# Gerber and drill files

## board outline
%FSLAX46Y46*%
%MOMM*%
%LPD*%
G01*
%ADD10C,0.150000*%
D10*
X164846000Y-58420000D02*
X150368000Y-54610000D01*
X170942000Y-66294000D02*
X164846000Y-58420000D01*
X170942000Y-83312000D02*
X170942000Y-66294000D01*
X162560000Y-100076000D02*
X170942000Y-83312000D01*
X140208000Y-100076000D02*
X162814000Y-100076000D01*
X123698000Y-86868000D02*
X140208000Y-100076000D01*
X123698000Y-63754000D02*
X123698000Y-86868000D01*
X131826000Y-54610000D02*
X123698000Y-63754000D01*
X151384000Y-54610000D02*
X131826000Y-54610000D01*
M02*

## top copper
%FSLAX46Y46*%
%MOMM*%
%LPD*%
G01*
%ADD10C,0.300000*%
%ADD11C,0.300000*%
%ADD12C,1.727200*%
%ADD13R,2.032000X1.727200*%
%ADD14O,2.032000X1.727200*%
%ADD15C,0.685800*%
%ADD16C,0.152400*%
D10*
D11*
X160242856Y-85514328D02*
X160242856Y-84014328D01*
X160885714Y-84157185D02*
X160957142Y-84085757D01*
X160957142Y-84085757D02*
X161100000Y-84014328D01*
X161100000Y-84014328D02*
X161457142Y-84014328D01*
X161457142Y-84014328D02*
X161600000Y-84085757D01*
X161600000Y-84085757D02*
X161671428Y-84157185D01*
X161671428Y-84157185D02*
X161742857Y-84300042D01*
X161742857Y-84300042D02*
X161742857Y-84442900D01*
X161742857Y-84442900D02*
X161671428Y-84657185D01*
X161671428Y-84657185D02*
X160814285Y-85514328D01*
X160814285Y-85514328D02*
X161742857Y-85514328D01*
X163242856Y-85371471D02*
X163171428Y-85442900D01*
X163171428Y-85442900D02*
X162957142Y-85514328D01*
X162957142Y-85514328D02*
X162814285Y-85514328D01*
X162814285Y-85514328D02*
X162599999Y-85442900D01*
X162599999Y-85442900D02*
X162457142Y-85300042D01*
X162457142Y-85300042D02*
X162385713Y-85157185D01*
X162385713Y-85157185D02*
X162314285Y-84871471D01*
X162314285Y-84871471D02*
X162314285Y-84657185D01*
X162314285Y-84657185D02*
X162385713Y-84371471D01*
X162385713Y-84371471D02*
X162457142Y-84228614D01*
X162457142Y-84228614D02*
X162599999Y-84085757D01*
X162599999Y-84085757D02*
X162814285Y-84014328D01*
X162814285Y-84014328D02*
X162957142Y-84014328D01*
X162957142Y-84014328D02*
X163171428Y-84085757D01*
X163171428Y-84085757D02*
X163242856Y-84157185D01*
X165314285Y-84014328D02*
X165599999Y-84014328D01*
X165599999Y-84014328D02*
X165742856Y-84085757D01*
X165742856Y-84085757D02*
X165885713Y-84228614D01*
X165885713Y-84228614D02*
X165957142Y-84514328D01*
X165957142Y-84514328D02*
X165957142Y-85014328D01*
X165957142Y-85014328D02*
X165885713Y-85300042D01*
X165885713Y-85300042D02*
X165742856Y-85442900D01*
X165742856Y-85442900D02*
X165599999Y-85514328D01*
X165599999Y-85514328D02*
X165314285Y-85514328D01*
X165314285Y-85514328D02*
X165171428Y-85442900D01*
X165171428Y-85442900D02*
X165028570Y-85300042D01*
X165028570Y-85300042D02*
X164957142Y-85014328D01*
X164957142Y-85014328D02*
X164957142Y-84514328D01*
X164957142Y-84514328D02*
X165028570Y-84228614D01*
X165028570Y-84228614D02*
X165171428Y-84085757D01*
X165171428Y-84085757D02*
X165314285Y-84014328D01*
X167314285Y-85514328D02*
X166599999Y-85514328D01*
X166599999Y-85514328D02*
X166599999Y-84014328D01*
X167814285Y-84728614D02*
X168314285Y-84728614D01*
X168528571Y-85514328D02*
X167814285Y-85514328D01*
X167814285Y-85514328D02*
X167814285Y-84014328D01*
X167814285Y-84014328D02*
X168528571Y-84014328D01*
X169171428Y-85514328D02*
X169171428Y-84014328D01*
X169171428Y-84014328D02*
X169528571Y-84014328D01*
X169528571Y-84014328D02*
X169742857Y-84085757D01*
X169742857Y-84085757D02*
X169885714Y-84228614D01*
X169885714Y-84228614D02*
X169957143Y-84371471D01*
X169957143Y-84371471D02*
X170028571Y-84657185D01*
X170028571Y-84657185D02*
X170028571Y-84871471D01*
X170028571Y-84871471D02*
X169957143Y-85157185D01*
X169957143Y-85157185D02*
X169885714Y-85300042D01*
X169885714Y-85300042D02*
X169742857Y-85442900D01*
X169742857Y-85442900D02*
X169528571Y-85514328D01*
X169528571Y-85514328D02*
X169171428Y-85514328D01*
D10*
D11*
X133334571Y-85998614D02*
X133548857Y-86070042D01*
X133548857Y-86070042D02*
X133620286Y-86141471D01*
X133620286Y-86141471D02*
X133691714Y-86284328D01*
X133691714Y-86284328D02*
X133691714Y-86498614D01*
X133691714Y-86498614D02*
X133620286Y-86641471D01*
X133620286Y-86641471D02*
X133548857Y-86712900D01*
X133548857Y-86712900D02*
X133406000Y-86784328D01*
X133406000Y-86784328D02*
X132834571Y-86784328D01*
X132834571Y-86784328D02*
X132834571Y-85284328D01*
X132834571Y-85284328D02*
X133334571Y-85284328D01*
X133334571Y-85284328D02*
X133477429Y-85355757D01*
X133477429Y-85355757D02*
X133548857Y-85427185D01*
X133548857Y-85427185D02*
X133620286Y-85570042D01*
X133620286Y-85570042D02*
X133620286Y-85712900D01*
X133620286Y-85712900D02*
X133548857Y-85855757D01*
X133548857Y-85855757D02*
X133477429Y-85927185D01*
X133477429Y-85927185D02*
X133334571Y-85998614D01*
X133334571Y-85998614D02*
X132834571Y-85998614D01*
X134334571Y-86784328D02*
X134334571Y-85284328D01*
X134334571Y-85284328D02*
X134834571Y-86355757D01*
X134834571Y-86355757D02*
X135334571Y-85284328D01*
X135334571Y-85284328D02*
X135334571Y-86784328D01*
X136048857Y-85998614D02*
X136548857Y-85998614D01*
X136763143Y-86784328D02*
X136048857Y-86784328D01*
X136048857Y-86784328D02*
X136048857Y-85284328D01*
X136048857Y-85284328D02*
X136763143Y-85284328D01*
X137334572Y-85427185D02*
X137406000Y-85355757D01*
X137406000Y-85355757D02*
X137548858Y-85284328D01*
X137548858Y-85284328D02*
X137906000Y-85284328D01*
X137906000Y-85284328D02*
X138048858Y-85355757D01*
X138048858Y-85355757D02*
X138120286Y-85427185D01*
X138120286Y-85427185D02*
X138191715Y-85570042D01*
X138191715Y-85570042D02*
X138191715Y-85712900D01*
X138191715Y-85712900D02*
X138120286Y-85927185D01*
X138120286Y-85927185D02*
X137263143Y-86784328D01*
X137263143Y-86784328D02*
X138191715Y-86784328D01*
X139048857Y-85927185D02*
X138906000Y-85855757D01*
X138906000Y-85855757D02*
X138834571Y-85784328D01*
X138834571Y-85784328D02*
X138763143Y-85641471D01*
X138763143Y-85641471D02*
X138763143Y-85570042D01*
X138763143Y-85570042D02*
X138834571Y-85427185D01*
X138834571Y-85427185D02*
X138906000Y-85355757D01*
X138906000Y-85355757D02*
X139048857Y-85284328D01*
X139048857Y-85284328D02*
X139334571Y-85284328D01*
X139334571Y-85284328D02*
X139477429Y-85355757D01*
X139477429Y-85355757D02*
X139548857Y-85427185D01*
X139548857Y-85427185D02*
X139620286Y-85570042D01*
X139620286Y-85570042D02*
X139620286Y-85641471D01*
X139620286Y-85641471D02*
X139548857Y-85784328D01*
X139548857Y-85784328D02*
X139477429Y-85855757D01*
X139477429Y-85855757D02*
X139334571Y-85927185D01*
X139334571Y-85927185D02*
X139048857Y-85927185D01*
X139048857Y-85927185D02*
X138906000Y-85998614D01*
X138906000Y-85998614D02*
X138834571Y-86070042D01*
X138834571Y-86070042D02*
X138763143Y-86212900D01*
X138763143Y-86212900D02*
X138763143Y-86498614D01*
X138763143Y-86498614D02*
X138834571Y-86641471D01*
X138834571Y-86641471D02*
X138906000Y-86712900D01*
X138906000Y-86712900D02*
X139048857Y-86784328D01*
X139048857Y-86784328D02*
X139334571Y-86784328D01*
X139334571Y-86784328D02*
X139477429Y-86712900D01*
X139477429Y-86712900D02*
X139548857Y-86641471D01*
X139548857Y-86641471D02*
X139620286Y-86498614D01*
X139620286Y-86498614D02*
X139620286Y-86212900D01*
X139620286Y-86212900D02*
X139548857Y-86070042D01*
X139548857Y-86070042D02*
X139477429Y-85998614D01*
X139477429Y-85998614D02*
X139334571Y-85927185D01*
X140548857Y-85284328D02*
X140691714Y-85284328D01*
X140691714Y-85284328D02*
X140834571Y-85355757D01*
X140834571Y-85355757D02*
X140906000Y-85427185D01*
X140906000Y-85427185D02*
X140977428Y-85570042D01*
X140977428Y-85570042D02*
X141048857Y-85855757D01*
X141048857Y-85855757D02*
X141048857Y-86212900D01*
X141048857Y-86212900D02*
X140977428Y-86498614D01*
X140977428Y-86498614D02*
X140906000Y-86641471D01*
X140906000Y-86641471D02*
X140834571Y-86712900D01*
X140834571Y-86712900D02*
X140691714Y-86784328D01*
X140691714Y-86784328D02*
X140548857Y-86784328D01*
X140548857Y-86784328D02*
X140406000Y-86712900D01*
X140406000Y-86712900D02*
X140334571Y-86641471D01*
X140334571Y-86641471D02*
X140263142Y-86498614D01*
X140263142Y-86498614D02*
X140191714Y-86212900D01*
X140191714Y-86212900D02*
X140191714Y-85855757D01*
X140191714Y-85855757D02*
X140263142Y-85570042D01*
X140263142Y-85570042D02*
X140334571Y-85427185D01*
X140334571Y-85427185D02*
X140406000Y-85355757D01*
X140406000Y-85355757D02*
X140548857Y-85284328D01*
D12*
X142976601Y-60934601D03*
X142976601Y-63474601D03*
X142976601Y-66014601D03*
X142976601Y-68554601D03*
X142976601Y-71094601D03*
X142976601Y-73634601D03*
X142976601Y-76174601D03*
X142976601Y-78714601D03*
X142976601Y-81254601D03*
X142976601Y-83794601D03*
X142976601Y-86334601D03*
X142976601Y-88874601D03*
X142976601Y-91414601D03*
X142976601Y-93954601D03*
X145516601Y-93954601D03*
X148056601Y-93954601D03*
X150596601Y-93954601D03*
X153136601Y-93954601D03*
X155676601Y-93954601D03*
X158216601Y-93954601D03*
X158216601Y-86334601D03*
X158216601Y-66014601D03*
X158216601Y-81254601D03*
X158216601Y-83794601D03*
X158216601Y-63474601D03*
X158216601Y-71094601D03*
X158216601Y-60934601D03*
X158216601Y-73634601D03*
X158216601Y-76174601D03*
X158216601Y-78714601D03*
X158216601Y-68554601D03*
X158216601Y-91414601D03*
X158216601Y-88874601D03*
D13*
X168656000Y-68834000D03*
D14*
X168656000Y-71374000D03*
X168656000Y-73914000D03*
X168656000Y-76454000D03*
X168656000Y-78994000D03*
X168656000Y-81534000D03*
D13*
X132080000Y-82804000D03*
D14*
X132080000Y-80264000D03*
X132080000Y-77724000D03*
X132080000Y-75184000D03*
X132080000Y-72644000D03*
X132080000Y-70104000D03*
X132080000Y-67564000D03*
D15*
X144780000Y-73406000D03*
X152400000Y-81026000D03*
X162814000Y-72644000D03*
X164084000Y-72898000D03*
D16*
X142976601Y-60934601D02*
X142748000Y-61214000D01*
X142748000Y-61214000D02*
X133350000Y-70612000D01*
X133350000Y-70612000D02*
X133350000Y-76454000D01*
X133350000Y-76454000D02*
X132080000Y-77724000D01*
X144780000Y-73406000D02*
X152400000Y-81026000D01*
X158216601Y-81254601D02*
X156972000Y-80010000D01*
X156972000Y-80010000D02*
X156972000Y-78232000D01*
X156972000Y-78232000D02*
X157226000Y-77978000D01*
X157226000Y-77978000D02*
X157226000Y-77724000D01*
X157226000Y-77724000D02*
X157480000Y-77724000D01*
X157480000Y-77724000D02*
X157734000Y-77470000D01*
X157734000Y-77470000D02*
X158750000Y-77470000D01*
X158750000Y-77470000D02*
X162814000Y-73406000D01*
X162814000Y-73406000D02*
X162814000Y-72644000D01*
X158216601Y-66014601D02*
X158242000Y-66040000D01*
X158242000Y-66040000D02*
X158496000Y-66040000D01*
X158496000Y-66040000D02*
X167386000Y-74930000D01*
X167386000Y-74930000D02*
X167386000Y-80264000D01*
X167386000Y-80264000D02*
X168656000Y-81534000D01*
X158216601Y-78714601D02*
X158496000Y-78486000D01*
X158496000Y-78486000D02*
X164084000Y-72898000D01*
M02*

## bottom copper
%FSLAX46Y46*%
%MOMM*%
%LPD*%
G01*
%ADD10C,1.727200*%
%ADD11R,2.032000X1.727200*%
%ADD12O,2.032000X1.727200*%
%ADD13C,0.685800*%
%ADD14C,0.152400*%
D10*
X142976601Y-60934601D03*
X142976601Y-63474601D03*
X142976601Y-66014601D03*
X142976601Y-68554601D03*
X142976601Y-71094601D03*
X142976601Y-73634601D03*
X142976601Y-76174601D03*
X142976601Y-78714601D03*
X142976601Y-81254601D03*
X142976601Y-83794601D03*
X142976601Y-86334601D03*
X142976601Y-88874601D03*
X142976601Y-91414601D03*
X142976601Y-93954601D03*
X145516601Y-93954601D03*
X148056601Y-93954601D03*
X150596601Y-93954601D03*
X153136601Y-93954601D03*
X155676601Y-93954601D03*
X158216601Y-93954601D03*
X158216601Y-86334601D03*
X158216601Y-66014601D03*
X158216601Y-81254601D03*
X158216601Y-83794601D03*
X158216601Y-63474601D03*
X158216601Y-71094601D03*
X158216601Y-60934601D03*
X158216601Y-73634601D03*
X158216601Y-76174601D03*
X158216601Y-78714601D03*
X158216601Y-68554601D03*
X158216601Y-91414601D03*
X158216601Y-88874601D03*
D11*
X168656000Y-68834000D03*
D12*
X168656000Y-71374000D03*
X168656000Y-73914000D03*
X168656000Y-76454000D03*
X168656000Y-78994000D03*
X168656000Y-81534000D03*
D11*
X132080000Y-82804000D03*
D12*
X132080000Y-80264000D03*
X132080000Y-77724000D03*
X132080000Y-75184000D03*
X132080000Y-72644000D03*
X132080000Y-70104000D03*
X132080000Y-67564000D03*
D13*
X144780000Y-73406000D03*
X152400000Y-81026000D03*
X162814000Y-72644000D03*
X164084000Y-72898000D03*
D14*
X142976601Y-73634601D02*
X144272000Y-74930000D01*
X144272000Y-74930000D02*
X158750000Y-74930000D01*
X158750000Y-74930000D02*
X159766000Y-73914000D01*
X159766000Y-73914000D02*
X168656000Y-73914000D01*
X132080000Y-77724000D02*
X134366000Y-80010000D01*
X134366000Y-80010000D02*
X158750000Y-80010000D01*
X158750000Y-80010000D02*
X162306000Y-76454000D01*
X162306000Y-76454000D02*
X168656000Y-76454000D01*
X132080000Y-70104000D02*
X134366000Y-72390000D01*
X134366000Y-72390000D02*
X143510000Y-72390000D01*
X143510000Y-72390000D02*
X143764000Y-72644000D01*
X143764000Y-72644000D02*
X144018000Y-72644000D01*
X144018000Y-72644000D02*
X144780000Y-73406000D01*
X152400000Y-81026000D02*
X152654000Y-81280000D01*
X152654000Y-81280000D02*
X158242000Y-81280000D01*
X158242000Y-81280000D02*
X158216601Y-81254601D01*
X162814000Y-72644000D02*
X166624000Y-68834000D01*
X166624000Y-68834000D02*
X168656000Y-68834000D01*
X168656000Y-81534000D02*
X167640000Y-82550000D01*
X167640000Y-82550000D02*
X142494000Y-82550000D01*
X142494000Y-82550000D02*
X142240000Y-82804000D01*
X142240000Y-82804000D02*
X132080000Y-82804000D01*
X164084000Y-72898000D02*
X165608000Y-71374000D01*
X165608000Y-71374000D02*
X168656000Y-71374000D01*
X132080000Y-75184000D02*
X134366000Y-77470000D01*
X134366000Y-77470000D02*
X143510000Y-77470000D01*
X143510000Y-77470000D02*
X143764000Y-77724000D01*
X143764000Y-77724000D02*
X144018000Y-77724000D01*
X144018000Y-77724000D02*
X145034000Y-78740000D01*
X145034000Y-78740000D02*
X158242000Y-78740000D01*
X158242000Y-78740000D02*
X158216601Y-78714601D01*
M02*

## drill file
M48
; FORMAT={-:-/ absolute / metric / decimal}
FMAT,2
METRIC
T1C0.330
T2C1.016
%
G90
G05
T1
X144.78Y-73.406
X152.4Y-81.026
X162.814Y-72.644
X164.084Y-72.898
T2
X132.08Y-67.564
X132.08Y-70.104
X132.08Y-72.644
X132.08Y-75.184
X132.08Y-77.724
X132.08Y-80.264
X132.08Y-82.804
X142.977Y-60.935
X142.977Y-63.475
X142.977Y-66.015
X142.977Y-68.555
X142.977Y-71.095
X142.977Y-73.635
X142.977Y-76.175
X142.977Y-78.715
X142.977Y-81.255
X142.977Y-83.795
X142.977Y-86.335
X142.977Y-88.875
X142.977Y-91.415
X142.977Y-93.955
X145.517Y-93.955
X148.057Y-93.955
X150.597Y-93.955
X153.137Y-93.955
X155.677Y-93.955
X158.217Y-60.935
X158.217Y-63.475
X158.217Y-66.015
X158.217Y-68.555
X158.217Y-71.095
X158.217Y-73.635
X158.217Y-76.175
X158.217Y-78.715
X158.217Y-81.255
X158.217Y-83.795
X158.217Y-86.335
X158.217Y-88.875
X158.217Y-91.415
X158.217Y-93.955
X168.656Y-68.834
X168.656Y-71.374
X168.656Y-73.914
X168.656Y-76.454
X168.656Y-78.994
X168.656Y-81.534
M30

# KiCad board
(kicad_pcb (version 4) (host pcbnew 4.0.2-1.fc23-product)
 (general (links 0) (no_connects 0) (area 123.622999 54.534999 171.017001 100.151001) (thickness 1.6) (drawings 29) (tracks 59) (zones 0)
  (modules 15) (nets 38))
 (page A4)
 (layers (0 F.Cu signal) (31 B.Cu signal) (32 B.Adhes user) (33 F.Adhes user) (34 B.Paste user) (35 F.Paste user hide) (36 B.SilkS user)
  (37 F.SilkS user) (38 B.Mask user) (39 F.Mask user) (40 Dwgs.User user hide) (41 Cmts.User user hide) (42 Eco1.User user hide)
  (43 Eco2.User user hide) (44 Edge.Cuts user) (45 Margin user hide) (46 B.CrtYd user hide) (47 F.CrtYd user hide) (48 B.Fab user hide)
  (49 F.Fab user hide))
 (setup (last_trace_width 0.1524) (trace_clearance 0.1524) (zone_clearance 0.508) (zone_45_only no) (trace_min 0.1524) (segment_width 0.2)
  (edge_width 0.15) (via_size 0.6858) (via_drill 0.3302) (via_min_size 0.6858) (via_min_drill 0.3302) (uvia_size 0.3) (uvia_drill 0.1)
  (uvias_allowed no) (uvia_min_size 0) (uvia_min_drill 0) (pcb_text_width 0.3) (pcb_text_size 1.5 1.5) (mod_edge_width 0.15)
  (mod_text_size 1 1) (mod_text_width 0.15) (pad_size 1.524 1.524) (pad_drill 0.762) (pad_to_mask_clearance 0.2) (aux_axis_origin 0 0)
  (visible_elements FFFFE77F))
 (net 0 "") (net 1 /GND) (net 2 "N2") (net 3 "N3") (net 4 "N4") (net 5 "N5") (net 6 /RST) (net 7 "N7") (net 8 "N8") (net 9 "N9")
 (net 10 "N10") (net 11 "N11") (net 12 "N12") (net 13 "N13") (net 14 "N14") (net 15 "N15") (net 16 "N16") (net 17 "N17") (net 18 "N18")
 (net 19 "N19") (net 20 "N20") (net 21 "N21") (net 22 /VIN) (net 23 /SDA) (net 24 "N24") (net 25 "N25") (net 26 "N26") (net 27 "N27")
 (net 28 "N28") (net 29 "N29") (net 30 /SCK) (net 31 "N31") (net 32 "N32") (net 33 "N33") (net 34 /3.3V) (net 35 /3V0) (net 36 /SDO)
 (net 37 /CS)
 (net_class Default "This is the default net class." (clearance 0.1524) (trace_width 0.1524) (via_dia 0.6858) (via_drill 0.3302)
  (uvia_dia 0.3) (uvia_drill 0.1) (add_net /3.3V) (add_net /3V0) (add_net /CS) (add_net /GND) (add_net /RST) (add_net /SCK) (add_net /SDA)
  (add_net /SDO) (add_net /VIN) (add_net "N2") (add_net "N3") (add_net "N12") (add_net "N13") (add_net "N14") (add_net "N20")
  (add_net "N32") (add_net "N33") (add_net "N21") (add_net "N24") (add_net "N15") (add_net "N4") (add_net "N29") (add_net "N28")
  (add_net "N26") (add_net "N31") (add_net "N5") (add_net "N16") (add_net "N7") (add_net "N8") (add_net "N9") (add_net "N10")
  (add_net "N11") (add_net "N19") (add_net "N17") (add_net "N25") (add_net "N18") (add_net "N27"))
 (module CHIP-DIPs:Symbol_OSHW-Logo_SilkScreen (layer B.Cu) (at 127.508 64.77 180)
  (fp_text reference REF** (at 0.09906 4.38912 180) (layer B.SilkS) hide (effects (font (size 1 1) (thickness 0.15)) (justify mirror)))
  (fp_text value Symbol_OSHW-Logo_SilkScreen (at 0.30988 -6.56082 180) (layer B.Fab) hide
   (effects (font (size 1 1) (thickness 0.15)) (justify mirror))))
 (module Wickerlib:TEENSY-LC (layer F.Cu) (at 153.136601 71.094601)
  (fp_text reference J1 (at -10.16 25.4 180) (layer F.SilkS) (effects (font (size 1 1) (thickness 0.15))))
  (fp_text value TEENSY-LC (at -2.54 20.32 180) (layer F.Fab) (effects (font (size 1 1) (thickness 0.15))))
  (pad G1 thru_hole circle (at -10.16 -10.16) (size 1.7272 1.7272) (drill 1.016) (layers *.Cu *.Mask F.SilkS) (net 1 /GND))
  (pad 0 thru_hole circle (at -10.16 -7.62) (size 1.7272 1.7272) (drill 1.016) (layers *.Cu *.Mask F.SilkS) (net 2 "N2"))
  (pad 1 thru_hole circle (at -10.16 -5.08) (size 1.7272 1.7272) (drill 1.016) (layers *.Cu *.Mask F.SilkS) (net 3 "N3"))
  (pad 2 thru_hole circle (at -10.16 -2.54) (size 1.7272 1.7272) (drill 1.016) (layers *.Cu *.Mask F.SilkS) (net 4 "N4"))
  (pad 3 thru_hole circle (at -10.16 0) (size 1.7272 1.7272) (drill 1.016) (layers *.Cu *.Mask F.SilkS) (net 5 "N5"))
  (pad 4 thru_hole circle (at -10.16 2.54) (size 1.7272 1.7272) (drill 1.016) (layers *.Cu *.Mask F.SilkS) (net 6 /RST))
  (pad 5 thru_hole circle (at -10.16 5.08) (size 1.7272 1.7272) (drill 1.016) (layers *.Cu *.Mask F.SilkS) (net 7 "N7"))
  (pad 6 thru_hole circle (at -10.16 7.62) (size 1.7272 1.7272) (drill 1.016) (layers *.Cu *.Mask F.SilkS) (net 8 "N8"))
  (pad 7 thru_hole circle (at -10.16 10.16) (size 1.7272 1.7272) (drill 1.016) (layers *.Cu *.Mask F.SilkS) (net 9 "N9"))
  (pad 8 thru_hole circle (at -10.16 12.7) (size 1.7272 1.7272) (drill 1.016) (layers *.Cu *.Mask F.SilkS) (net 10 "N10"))
  (pad 9 thru_hole circle (at -10.16 15.24) (size 1.7272 1.7272) (drill 1.016) (layers *.Cu *.Mask F.SilkS) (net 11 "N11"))
  (pad 10 thru_hole circle (at -10.16 17.78) (size 1.7272 1.7272) (drill 1.016) (layers *.Cu *.Mask F.SilkS) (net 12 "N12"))
  (pad 11 thru_hole circle (at -10.16 20.32) (size 1.7272 1.7272) (drill 1.016) (layers *.Cu *.Mask F.SilkS) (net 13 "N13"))
  (pad 12 thru_hole circle (at -10.16 22.86) (size 1.7272 1.7272) (drill 1.016) (layers *.Cu *.Mask F.SilkS) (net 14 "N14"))
  (pad 17A thru_hole circle (at -7.62 22.86) (size 1.7272 1.7272) (drill 1.016) (layers *.Cu *.Mask F.SilkS) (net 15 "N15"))
  (pad 3V1 thru_hole circle (at -5.08 22.86) (size 1.7272 1.7272) (drill 1.016) (layers *.Cu *.Mask F.SilkS) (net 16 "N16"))
  (pad G2 thru_hole circle (at -2.54 22.86) (size 1.7272 1.7272) (drill 1.016) (layers *.Cu *.Mask F.SilkS) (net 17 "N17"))
  (pad PGM thru_hole circle (at 0 22.86) (size 1.7272 1.7272) (drill 1.016) (layers *.Cu *.Mask F.SilkS) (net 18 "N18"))
  (pad DAC thru_hole circle (at 2.54 22.86) (size 1.7272 1.7272) (drill 1.016) (layers *.Cu *.Mask F.SilkS) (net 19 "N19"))
  (pad 13 thru_hole circle (at 5.08 22.86) (size 1.7272 1.7272) (drill 1.016) (layers *.Cu *.Mask F.SilkS) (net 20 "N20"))
  (pad 16 thru_hole circle (at 5.08 15.24) (size 1.7272 1.7272) (drill 1.016) (layers *.Cu *.Mask F.SilkS) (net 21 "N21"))
  (pad 3V2 thru_hole circle (at 5.08 -5.08) (size 1.7272 1.7272) (drill 1.016) (layers *.Cu *.Mask F.SilkS) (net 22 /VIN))
  (pad 18 thru_hole circle (at 5.08 10.16) (size 1.7272 1.7272) (drill 1.016) (layers *.Cu *.Mask F.SilkS) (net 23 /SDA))
  (pad 17 thru_hole circle (at 5.08 12.7) (size 1.7272 1.7272) (drill 1.016) (layers *.Cu *.Mask F.SilkS) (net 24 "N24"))
  (pad G3 thru_hole circle (at 5.08 -7.62) (size 1.7272 1.7272) (drill 1.016) (layers *.Cu *.Mask F.SilkS) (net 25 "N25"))
  (pad 22 thru_hole circle (at 5.08 0) (size 1.7272 1.7272) (drill 1.016) (layers *.Cu *.Mask F.SilkS) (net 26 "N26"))
  (pad VIN thru_hole circle (at 5.08 -10.16) (size 1.7272 1.7272) (drill 1.016) (layers *.Cu *.Mask F.SilkS) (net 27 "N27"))
  (pad 21 thru_hole circle (at 5.08 2.54) (size 1.7272 1.7272) (drill 1.016) (layers *.Cu *.Mask F.SilkS) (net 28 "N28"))
  (pad 20 thru_hole circle (at 5.08 5.08) (size 1.7272 1.7272) (drill 1.016) (layers *.Cu *.Mask F.SilkS) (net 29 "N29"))
  (pad 19 thru_hole circle (at 5.08 7.62) (size 1.7272 1.7272) (drill 1.016) (layers *.Cu *.Mask F.SilkS) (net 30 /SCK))
  (pad 23 thru_hole circle (at 5.08 -2.54) (size 1.7272 1.7272) (drill 1.016) (layers *.Cu *.Mask F.SilkS) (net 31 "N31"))
  (pad 14 thru_hole circle (at 5.08 20.32) (size 1.7272 1.7272) (drill 1.016) (layers *.Cu *.Mask F.SilkS) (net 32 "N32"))
  (pad 15 thru_hole circle (at 5.08 17.78) (size 1.7272 1.7272) (drill 1.016) (layers *.Cu *.Mask F.SilkS) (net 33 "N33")))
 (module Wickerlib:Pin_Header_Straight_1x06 (layer F.Cu) (at 168.656 68.834)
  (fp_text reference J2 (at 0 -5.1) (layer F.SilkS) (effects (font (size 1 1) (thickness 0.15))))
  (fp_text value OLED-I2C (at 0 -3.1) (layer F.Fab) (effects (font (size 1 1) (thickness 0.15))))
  (pad 1 thru_hole rect (at 0 0) (size 2.032 1.7272) (drill 1.016) (layers *.Cu *.Mask F.SilkS) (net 23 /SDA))
  (pad 2 thru_hole oval (at 0 2.54) (size 2.032 1.7272) (drill 1.016) (layers *.Cu *.Mask F.SilkS) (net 30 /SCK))
  (pad 3 thru_hole oval (at 0 5.08) (size 2.032 1.7272) (drill 1.016) (layers *.Cu *.Mask F.SilkS) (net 6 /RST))
  (pad 4 thru_hole oval (at 0 7.62) (size 2.032 1.7272) (drill 1.016) (layers *.Cu *.Mask F.SilkS) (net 1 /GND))
  (pad 5 thru_hole oval (at 0 10.16) (size 2.032 1.7272) (drill 1.016) (layers *.Cu *.Mask F.SilkS) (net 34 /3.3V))
  (pad 6 thru_hole oval (at 0 12.7) (size 2.032 1.7272) (drill 1.016) (layers *.Cu *.Mask F.SilkS) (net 22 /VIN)))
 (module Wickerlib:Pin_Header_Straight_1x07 (layer F.Cu) (at 132.08 82.804 180)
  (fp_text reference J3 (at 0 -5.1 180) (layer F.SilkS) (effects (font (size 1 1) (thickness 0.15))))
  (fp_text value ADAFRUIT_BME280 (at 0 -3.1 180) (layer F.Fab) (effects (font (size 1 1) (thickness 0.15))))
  (pad 1 thru_hole rect (at 0 0 180) (size 2.032 1.7272) (drill 1.016) (layers *.Cu *.Mask F.SilkS) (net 22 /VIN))
  (pad 2 thru_hole oval (at 0 2.54 180) (size 2.032 1.7272) (drill 1.016) (layers *.Cu *.Mask F.SilkS) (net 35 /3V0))
  (pad 3 thru_hole oval (at 0 5.08 180) (size 2.032 1.7272) (drill 1.016) (layers *.Cu *.Mask F.SilkS) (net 1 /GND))
  (pad 4 thru_hole oval (at 0 7.62 180) (size 2.032 1.7272) (drill 1.016) (layers *.Cu *.Mask F.SilkS) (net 30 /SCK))
  (pad 5 thru_hole oval (at 0 10.16 180) (size 2.032 1.7272) (drill 1.016) (layers *.Cu *.Mask F.SilkS) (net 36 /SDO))
  (pad 6 thru_hole oval (at 0 12.7 180) (size 2.032 1.7272) (drill 1.016) (layers *.Cu *.Mask F.SilkS) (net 23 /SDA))
  (pad 7 thru_hole oval (at 0 15.24 180) (size 2.032 1.7272) (drill 1.016) (layers *.Cu *.Mask F.SilkS) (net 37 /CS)))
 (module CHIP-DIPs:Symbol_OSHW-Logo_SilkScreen (layer F.Cu) (at 148.59 88.138 270)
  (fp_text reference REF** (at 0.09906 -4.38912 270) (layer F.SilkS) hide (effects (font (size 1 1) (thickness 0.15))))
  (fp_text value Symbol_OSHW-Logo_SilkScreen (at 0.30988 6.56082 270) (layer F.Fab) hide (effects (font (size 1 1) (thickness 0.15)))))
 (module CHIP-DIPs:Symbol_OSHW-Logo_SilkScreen (layer F.Cu) (at 148.59 88.138 270)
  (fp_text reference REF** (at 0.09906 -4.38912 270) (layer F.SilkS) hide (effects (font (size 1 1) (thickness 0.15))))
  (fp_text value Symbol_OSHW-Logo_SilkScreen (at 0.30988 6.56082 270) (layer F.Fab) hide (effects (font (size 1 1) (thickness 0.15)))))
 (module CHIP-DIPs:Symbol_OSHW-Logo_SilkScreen (layer F.Cu) (at 148.59 88.138 270)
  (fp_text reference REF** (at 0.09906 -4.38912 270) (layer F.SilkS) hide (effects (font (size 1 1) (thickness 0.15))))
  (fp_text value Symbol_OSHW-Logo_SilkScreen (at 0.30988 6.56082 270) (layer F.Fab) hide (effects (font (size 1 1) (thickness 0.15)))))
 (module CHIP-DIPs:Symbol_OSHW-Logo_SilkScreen (layer F.Cu) (at 137.414 91.186 270)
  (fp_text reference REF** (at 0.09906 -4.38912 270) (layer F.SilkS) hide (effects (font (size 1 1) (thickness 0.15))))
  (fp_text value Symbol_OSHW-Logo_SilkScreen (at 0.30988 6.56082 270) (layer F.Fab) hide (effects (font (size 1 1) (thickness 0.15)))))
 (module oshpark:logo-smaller (layer F.Cu) (at 149.098 104.14 270)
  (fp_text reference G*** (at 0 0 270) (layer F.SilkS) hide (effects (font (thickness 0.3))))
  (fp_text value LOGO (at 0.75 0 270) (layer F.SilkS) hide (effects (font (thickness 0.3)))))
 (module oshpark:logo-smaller (layer F.Cu) (at 149.352 77.47 270)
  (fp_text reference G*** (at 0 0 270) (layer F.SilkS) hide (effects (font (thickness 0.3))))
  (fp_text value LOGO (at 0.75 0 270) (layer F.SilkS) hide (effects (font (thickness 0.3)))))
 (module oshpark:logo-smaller (layer F.Cu) (at 149.352 77.47 270)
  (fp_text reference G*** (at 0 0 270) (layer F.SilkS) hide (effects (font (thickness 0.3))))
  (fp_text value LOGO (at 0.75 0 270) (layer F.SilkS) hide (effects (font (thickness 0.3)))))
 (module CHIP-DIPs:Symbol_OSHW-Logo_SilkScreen (layer B.Cu) (at 133.604 62.484)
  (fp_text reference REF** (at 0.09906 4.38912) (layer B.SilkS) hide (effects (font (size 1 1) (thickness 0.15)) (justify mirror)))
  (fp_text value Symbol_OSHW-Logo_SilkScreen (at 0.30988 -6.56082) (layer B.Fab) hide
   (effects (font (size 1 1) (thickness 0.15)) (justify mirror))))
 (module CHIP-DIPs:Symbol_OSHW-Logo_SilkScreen (layer F.Cu) (at 133.604 62.484)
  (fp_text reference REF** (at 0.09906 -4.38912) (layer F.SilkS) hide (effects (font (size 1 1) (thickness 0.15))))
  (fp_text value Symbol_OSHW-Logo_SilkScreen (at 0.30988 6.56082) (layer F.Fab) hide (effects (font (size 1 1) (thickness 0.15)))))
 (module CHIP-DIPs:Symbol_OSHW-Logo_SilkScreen (layer F.Cu) (at 133.604 62.484)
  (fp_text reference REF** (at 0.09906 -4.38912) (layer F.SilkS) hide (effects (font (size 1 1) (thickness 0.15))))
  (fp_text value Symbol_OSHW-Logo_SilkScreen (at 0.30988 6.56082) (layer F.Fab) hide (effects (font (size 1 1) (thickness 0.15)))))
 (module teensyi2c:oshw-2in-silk (layer B.Cu) (at 148.59 75.438 90)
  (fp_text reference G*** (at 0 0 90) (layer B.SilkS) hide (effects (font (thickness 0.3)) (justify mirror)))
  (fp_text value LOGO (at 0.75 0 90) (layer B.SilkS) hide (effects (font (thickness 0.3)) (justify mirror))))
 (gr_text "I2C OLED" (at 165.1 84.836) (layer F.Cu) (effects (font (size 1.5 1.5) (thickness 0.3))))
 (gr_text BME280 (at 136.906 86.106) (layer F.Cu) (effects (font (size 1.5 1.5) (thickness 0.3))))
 (gr_line (start 164.846 58.42) (end 150.368 54.61) (layer Edge.Cuts) (width 0.15))
 (gr_line (start 170.942 66.294) (end 164.846 58.42) (layer Edge.Cuts) (width 0.15))
 (gr_line (start 170.942 83.312) (end 170.942 66.294) (layer Edge.Cuts) (width 0.15))
 (gr_line (start 162.56 100.076) (end 170.942 83.312) (layer Edge.Cuts) (width 0.15))
 (gr_line (start 140.208 100.076) (end 162.814 100.076) (layer Edge.Cuts) (width 0.15))
 (gr_line (start 123.698 86.868) (end 140.208 100.076) (layer Edge.Cuts) (width 0.15))
 (gr_line (start 123.698 63.754) (end 123.698 86.868) (layer Edge.Cuts) (width 0.15))
 (gr_line (start 131.826 54.61) (end 123.698 63.754) (layer Edge.Cuts) (width 0.15))
 (gr_line (start 151.384 54.61) (end 131.826 54.61) (layer Edge.Cuts) (width 0.15))
 (segment (start 132.08 52.07) (end 105.664 52.07) (width 0.1524) (layer Dwgs.User) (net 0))
 (segment (start 133.096 57.658) (end 124.206 66.548) (width 0.1524) (layer Dwgs.User) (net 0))
 (segment (start 144.78 57.658) (end 133.096 57.658) (width 0.1524) (layer Dwgs.User) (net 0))
 (segment (start 142.976601 73.634601) (end 144.272 74.93) (width 0.1524) (layer B.Cu) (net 6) (status 80000))
 (segment (start 144.272 74.93) (end 158.75 74.93) (width 0.1524) (layer B.Cu) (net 6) (status 80000))
 (segment (start 158.75 74.93) (end 159.766 73.914) (width 0.1524) (layer B.Cu) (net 6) (status 80000))
 (segment (start 159.766 73.914) (end 168.656 73.914) (width 0.1524) (layer B.Cu) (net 6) (status 80000))
 (segment (start 142.976601 60.934601) (end 142.748 61.214) (width 0.1524) (layer F.Cu) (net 1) (status 80000))
 (segment (start 142.748 61.214) (end 133.35 70.612) (width 0.1524) (layer F.Cu) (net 1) (status 80000))
 (segment (start 133.35 70.612) (end 133.35 76.454) (width 0.1524) (layer F.Cu) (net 1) (status 80000))
 (segment (start 133.35 76.454) (end 132.08 77.724) (width 0.1524) (layer F.Cu) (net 1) (status 80000))
 (segment (start 132.08 77.724) (end 134.366 80.01) (width 0.1524) (layer B.Cu) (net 1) (status 80000))
 (segment (start 134.366 80.01) (end 158.75 80.01) (width 0.1524) (layer B.Cu) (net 1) (status 80000))
 (segment (start 158.75 80.01) (end 162.306 76.454) (width 0.1524) (layer B.Cu) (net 1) (status 80000))
 (segment (start 162.306 76.454) (end 168.656 76.454) (width 0.1524) (layer B.Cu) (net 1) (status 80000))
 (segment (start 132.08 70.104) (end 134.366 72.39) (width 0.1524) (layer B.Cu) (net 23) (status 80000))
 (segment (start 134.366 72.39) (end 143.51 72.39) (width 0.1524) (layer B.Cu) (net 23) (status 80000))
 (segment (start 143.51 72.39) (end 143.764 72.644) (width 0.1524) (layer B.Cu) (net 23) (status 80000))
 (segment (start 143.764 72.644) (end 144.018 72.644) (width 0.1524) (layer B.Cu) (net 23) (status 80000))
 (segment (start 144.018 72.644) (end 144.78 73.406) (width 0.1524) (layer B.Cu) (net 23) (status 80000))
 (via (at 144.78 73.406) (size 0.6858) (layers F.Cu B.Cu) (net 23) (status 80000))
 (segment (start 144.78 73.406) (end 152.4 81.026) (width 0.1524) (layer F.Cu) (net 23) (status 80000))
 (via (at 152.4 81.026) (size 0.6858) (layers F.Cu B.Cu) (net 23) (status 80000))
 (segment (start 152.4 81.026) (end 152.654 81.28) (width 0.1524) (layer B.Cu) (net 23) (status 80000))
 (segment (start 152.654 81.28) (end 158.242 81.28) (width 0.1524) (layer B.Cu) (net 23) (status 80000))
 (segment (start 158.242 81.28) (end 158.216601 81.254601) (width 0.1524) (layer B.Cu) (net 23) (status 80000))
 (segment (start 158.216601 81.254601) (end 156.972 80.01) (width 0.1524) (layer F.Cu) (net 23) (status 80000))
 (segment (start 156.972 80.01) (end 156.972 78.232) (width 0.1524) (layer F.Cu) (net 23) (status 80000))
 (segment (start 156.972 78.232) (end 157.226 77.978) (width 0.1524) (layer F.Cu) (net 23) (status 80000))
 (segment (start 157.226 77.978) (end 157.226 77.724) (width 0.1524) (layer F.Cu) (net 23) (status 80000))
 (segment (start 157.226 77.724) (end 157.48 77.724) (width 0.1524) (layer F.Cu) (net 23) (status 80000))
 (segment (start 157.48 77.724) (end 157.734 77.47) (width 0.1524) (layer F.Cu) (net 23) (status 80000))
 (segment (start 157.734 77.47) (end 158.75 77.47) (width 0.1524) (layer F.Cu) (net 23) (status 80000))
 (segment (start 158.75 77.47) (end 162.814 73.406) (width 0.1524) (layer F.Cu) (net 23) (status 80000))
 (segment (start 162.814 73.406) (end 162.814 72.644) (width 0.1524) (layer F.Cu) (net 23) (status 80000))
 (via (at 162.814 72.644) (size 0.6858) (layers F.Cu B.Cu) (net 23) (status 80000))
 (segment (start 162.814 72.644) (end 166.624 68.834) (width 0.1524) (layer B.Cu) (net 23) (status 80000))
 (segment (start 166.624 68.834) (end 168.656 68.834) (width 0.1524) (layer B.Cu) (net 23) (status 80000))
 (segment (start 158.216601 66.014601) (end 158.242 66.04) (width 0.1524) (layer F.Cu) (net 22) (status 80000))
 (segment (start 158.242 66.04) (end 158.496 66.04) (width 0.1524) (layer F.Cu) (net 22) (status 80000))
 (segment (start 158.496 66.04) (end 167.386 74.93) (width 0.1524) (layer F.Cu) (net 22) (status 80000))
 (segment (start 167.386 74.93) (end 167.386 80.264) (width 0.1524) (layer F.Cu) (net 22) (status 80000))
 (segment (start 167.386 80.264) (end 168.656 81.534) (width 0.1524) (layer F.Cu) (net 22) (status 80000))
 (segment (start 168.656 81.534) (end 167.64 82.55) (width 0.1524) (layer B.Cu) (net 22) (status 80000))
 (segment (start 167.64 82.55) (end 142.494 82.55) (width 0.1524) (layer B.Cu) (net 22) (status 80000))
 (segment (start 142.494 82.55) (end 142.24 82.804) (width 0.1524) (layer B.Cu) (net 22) (status 80000))
 (segment (start 142.24 82.804) (end 132.08 82.804) (width 0.1524) (layer B.Cu) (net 22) (status 80000))
 (segment (start 158.216601 78.714601) (end 158.496 78.486) (width 0.1524) (layer F.Cu) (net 30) (status 80000))
 (segment (start 158.496 78.486) (end 164.084 72.898) (width 0.1524) (layer F.Cu) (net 30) (status 80000))
 (via (at 164.084 72.898) (size 0.6858) (layers F.Cu B.Cu) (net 30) (status 80000))
 (segment (start 164.084 72.898) (end 165.608 71.374) (width 0.1524) (layer B.Cu) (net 30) (status 80000))
 (segment (start 165.608 71.374) (end 168.656 71.374) (width 0.1524) (layer B.Cu) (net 30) (status 80000))
 (segment (start 132.08 75.184) (end 134.366 77.47) (width 0.1524) (layer B.Cu) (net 30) (status 80000))
 (segment (start 134.366 77.47) (end 143.51 77.47) (width 0.1524) (layer B.Cu) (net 30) (status 80000))
 (segment (start 143.51 77.47) (end 143.764 77.724) (width 0.1524) (layer B.Cu) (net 30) (status 80000))
 (segment (start 143.764 77.724) (end 144.018 77.724) (width 0.1524) (layer B.Cu) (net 30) (status 80000))
 (segment (start 144.018 77.724) (end 145.034 78.74) (width 0.1524) (layer B.Cu) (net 30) (status 80000))
 (segment (start 145.034 78.74) (end 158.242 78.74) (width 0.1524) (layer B.Cu) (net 30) (status 80000))
 (segment (start 158.242 78.74) (end 158.216601 78.714601) (width 0.1524) (layer B.Cu) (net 30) (status 80000)))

